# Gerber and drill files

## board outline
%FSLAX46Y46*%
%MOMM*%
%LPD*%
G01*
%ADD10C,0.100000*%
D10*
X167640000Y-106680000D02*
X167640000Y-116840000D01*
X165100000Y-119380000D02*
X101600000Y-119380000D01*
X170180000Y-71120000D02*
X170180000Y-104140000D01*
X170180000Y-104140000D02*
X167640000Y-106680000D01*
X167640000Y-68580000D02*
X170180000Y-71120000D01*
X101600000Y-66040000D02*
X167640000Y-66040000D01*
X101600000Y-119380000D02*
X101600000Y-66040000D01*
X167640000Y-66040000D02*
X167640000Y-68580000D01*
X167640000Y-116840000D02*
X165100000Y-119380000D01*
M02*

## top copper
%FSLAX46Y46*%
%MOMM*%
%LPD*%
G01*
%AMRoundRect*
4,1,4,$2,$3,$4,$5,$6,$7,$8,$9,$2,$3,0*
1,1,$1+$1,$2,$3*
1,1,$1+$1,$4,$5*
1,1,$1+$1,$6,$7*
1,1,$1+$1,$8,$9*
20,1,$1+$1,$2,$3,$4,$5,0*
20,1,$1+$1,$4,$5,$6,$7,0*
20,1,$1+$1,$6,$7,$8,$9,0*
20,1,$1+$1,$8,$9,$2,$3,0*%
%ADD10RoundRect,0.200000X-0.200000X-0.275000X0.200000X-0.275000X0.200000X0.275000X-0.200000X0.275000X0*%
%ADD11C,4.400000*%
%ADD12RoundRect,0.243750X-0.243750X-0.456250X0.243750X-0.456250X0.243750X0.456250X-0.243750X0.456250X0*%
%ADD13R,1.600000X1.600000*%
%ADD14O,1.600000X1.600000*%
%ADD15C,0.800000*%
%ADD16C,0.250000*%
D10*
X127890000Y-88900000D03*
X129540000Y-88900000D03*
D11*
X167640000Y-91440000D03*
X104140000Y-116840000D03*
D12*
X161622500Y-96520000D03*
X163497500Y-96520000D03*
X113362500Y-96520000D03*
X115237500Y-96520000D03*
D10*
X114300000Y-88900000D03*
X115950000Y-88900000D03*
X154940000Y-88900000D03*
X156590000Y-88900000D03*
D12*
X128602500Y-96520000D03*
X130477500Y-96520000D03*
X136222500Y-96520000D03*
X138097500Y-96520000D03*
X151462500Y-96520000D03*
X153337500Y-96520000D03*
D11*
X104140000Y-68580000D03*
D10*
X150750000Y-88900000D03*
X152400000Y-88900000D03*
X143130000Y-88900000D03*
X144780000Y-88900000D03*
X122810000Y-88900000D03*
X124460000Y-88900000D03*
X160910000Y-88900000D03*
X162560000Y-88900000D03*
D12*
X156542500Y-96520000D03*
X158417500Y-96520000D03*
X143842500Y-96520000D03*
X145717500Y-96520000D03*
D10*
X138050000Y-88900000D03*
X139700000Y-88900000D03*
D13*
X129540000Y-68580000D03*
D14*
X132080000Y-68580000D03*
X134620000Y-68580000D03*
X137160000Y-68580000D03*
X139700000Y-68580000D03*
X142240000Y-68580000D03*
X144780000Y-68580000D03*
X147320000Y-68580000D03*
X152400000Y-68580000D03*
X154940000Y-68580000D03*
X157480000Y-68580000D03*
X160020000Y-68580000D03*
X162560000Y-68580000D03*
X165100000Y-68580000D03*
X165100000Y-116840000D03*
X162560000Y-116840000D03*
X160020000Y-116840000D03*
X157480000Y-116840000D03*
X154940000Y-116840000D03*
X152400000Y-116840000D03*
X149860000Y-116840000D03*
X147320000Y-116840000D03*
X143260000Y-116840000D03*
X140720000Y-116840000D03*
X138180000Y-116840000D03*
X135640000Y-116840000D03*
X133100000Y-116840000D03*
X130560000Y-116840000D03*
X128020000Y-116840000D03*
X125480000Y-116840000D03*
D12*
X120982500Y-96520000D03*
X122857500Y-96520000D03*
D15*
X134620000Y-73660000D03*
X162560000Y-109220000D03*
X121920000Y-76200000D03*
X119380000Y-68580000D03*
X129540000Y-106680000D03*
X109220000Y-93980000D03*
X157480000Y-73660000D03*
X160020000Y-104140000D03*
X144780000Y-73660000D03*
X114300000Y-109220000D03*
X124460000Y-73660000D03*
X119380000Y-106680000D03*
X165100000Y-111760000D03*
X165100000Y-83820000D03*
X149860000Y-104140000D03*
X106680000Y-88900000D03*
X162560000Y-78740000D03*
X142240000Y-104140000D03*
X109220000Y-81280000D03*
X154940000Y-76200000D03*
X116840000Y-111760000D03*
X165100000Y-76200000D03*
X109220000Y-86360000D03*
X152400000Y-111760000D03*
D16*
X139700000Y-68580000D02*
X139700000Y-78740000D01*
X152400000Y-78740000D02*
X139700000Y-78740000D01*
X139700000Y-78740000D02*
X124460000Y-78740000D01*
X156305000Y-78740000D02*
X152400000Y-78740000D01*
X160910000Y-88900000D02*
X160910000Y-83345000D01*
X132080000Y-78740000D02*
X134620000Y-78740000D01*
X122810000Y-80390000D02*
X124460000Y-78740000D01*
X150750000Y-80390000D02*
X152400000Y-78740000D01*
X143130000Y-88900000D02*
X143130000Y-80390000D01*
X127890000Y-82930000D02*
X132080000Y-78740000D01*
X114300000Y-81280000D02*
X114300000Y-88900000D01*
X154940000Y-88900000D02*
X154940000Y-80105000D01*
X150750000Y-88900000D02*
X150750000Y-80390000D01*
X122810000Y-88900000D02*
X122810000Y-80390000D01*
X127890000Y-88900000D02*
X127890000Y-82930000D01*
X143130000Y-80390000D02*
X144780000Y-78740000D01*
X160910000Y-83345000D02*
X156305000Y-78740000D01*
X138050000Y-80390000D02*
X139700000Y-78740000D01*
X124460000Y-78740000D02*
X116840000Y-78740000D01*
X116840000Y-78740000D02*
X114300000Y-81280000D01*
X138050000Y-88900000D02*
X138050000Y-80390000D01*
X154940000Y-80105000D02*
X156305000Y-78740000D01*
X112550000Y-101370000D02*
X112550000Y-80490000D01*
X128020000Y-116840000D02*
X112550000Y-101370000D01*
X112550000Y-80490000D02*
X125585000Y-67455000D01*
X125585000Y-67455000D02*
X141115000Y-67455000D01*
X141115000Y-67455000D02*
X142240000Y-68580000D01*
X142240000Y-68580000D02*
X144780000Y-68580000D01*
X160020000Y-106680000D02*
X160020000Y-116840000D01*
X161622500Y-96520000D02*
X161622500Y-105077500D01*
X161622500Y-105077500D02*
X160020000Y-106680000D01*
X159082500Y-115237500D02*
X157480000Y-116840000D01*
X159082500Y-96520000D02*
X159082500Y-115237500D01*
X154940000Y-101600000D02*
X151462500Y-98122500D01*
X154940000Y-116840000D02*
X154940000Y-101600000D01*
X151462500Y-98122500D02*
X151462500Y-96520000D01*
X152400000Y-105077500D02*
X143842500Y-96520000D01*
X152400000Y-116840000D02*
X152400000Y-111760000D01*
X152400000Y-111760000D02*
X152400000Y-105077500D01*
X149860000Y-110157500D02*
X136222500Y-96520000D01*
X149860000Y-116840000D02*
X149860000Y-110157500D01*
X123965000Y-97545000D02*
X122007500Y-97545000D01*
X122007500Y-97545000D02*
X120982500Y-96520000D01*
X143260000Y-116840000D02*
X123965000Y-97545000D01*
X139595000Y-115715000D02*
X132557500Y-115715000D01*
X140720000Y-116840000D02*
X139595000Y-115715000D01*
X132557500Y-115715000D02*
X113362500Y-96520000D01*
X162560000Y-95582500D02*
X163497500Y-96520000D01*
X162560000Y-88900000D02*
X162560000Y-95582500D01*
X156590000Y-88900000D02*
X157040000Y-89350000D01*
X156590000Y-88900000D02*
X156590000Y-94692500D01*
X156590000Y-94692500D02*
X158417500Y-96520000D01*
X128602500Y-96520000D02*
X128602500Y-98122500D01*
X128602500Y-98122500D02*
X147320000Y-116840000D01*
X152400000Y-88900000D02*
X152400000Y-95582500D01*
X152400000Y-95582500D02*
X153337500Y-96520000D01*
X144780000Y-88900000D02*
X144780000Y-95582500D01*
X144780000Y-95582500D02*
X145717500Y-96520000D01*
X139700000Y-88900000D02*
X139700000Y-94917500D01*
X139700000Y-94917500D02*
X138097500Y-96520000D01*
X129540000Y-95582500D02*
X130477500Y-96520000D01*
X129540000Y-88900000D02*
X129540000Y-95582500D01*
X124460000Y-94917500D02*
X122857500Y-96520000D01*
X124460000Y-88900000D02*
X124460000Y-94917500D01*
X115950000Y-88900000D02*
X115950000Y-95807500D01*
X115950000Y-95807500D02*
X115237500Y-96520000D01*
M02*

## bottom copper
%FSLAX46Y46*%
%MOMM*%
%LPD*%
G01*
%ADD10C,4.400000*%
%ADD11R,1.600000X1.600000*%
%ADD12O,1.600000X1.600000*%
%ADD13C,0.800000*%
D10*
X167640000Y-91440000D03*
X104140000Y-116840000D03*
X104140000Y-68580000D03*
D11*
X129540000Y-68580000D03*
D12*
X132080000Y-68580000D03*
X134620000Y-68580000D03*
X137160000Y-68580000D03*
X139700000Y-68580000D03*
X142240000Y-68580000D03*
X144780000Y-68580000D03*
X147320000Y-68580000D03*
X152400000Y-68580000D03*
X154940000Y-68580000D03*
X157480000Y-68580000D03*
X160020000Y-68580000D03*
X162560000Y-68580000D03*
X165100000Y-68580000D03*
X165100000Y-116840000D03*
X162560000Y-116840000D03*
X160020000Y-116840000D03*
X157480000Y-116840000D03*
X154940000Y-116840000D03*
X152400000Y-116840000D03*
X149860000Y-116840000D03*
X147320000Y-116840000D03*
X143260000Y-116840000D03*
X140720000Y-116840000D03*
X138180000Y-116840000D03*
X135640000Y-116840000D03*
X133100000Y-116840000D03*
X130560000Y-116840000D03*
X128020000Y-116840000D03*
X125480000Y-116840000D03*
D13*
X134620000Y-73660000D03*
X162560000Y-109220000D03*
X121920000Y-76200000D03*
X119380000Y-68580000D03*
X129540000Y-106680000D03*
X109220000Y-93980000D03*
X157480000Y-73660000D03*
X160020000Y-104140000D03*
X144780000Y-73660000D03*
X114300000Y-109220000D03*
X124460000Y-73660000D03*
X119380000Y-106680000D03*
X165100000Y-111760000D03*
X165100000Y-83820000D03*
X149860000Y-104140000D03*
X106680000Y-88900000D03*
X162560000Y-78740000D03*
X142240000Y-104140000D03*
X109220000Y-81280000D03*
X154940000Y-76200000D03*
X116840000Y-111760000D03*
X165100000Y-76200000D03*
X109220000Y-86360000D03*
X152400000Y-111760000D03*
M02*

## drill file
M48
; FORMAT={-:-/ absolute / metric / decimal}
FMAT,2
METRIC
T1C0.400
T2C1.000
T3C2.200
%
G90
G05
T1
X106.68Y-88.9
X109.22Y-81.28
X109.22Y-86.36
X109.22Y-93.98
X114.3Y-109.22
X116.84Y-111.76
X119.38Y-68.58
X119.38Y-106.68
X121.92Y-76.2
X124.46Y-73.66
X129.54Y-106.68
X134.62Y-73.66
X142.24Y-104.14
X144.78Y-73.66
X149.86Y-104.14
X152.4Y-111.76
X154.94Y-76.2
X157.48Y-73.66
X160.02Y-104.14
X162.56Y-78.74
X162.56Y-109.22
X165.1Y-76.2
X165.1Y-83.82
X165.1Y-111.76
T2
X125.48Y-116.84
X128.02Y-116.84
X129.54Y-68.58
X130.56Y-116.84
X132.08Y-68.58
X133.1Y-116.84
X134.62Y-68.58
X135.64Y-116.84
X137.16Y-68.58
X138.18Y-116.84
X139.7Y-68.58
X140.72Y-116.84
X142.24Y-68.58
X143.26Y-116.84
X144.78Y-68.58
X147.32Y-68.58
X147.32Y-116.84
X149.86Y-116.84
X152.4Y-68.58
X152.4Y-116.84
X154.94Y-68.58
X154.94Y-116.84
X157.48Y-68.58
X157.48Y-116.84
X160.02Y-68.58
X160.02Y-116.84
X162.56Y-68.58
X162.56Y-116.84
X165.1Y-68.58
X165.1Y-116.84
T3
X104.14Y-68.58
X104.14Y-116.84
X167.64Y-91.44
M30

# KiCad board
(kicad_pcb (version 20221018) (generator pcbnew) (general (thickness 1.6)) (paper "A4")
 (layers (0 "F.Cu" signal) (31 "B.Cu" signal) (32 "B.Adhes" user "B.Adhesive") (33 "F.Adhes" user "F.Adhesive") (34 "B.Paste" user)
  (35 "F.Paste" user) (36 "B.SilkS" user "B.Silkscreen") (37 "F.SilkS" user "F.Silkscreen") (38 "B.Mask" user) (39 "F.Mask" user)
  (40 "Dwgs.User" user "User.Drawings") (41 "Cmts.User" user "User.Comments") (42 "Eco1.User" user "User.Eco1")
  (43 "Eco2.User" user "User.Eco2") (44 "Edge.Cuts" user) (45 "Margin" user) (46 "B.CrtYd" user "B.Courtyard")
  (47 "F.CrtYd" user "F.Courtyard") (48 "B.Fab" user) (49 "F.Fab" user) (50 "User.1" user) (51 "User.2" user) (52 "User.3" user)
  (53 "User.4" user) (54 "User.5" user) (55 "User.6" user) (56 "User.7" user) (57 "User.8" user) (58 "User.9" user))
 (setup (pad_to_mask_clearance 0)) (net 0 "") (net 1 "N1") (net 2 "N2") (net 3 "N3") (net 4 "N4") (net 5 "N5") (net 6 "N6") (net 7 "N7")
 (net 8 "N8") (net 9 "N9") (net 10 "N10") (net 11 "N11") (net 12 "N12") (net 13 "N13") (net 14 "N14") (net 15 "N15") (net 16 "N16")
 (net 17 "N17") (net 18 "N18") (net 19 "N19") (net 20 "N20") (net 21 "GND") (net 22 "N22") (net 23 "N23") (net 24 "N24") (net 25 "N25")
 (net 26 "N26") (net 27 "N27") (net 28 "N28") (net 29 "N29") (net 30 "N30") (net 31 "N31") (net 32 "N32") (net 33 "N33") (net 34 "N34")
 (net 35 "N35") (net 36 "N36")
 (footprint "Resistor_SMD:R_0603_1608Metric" (layer "F.Cu") (at 128.715 88.9)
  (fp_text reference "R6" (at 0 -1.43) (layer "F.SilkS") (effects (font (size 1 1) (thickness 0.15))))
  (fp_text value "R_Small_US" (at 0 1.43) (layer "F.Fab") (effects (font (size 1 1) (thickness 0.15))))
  (pad "1" smd roundrect (at -0.825 0) (size 0.8 0.95) (layers "F.Cu" "F.Paste" "F.Mask") (roundrect_rratio 0.25) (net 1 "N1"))
  (pad "2" smd roundrect (at 0.825 0) (size 0.8 0.95) (layers "F.Cu" "F.Paste" "F.Mask") (roundrect_rratio 0.25) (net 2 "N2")))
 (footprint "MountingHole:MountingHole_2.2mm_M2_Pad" (layer "F.Cu") (at 167.64 91.44)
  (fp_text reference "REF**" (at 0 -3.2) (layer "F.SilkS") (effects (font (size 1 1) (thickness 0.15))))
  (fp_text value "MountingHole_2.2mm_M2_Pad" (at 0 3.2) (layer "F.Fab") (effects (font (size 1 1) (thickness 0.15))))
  (pad "1" thru_hole circle (at 0 0) (size 4.4 4.4) (drill 2.2) (layers "*.Cu" "*.Mask")))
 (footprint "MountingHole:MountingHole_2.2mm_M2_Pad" (layer "F.Cu") (at 104.14 116.84)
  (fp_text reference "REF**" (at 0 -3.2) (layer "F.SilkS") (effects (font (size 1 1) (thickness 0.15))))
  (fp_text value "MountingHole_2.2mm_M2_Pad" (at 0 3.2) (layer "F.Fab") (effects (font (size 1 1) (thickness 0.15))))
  (pad "1" thru_hole circle (at 0 0) (size 4.4 4.4) (drill 2.2) (layers "*.Cu" "*.Mask")))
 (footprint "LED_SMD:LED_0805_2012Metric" (layer "F.Cu") (at 162.56 96.52)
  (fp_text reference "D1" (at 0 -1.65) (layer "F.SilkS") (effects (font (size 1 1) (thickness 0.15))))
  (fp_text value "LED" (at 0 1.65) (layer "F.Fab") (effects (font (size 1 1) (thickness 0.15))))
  (pad "1" smd roundrect (at -0.9375 0) (size 0.975 1.4) (layers "F.Cu" "F.Paste" "F.Mask") (roundrect_rratio 0.25) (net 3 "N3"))
  (pad "2" smd roundrect (at 0.9375 0) (size 0.975 1.4) (layers "F.Cu" "F.Paste" "F.Mask") (roundrect_rratio 0.25) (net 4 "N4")))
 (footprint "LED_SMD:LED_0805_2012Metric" (layer "F.Cu") (at 114.3 96.52)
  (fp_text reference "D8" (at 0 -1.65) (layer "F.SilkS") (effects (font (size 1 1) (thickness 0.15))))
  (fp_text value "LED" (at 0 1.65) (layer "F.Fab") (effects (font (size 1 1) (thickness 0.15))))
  (pad "1" smd roundrect (at -0.9375 0) (size 0.975 1.4) (layers "F.Cu" "F.Paste" "F.Mask") (roundrect_rratio 0.25) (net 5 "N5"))
  (pad "2" smd roundrect (at 0.9375 0) (size 0.975 1.4) (layers "F.Cu" "F.Paste" "F.Mask") (roundrect_rratio 0.25) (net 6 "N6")))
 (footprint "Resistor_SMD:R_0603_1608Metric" (layer "F.Cu") (at 115.125 88.9)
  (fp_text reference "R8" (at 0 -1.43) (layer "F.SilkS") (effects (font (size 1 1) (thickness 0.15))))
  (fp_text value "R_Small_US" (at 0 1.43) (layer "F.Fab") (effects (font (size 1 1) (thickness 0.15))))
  (pad "1" smd roundrect (at -0.825 0) (size 0.8 0.95) (layers "F.Cu" "F.Paste" "F.Mask") (roundrect_rratio 0.25) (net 1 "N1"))
  (pad "2" smd roundrect (at 0.825 0) (size 0.8 0.95) (layers "F.Cu" "F.Paste" "F.Mask") (roundrect_rratio 0.25) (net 6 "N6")))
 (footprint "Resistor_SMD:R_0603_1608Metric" (layer "F.Cu") (at 155.765 88.9)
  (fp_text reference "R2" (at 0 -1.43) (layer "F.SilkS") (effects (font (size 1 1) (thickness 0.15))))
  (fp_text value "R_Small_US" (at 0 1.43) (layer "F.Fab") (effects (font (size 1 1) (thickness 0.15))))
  (pad "1" smd roundrect (at -0.825 0) (size 0.8 0.95) (layers "F.Cu" "F.Paste" "F.Mask") (roundrect_rratio 0.25) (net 1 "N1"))
  (pad "2" smd roundrect (at 0.825 0) (size 0.8 0.95) (layers "F.Cu" "F.Paste" "F.Mask") (roundrect_rratio 0.25) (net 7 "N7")))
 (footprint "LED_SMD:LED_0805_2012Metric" (layer "F.Cu") (at 129.54 96.52)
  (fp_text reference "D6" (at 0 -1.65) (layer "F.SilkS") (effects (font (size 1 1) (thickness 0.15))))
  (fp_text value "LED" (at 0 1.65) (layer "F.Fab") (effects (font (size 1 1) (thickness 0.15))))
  (pad "1" smd roundrect (at -0.9375 0) (size 0.975 1.4) (layers "F.Cu" "F.Paste" "F.Mask") (roundrect_rratio 0.25) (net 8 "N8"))
  (pad "2" smd roundrect (at 0.9375 0) (size 0.975 1.4) (layers "F.Cu" "F.Paste" "F.Mask") (roundrect_rratio 0.25) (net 2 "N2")))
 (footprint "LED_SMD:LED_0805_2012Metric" (layer "F.Cu") (at 137.16 96.52)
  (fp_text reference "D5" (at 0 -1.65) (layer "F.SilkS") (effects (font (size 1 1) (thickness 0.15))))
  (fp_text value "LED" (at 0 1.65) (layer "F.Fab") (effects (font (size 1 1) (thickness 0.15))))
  (pad "1" smd roundrect (at -0.9375 0) (size 0.975 1.4) (layers "F.Cu" "F.Paste" "F.Mask") (roundrect_rratio 0.25) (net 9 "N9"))
  (pad "2" smd roundrect (at 0.9375 0) (size 0.975 1.4) (layers "F.Cu" "F.Paste" "F.Mask") (roundrect_rratio 0.25) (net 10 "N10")))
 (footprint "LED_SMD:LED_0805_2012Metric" (layer "F.Cu") (at 152.4 96.52)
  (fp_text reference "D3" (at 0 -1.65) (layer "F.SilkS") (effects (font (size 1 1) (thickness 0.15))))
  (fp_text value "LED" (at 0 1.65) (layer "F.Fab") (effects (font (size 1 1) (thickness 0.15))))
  (pad "1" smd roundrect (at -0.9375 0) (size 0.975 1.4) (layers "F.Cu" "F.Paste" "F.Mask") (roundrect_rratio 0.25) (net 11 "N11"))
  (pad "2" smd roundrect (at 0.9375 0) (size 0.975 1.4) (layers "F.Cu" "F.Paste" "F.Mask") (roundrect_rratio 0.25) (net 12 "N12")))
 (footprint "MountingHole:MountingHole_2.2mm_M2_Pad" (layer "F.Cu") (at 104.14 68.58)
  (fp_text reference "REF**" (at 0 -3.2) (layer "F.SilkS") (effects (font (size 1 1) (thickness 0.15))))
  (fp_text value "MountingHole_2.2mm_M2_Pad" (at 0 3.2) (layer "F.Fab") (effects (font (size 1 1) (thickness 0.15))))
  (pad "1" thru_hole circle (at 0 0) (size 4.4 4.4) (drill 2.2) (layers "*.Cu" "*.Mask")))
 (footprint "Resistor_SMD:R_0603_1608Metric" (layer "F.Cu") (at 151.575 88.9)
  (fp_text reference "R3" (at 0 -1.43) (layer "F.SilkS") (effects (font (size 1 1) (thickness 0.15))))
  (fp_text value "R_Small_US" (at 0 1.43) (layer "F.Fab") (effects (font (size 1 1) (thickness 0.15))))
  (pad "1" smd roundrect (at -0.825 0) (size 0.8 0.95) (layers "F.Cu" "F.Paste" "F.Mask") (roundrect_rratio 0.25) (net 1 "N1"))
  (pad "2" smd roundrect (at 0.825 0) (size 0.8 0.95) (layers "F.Cu" "F.Paste" "F.Mask") (roundrect_rratio 0.25) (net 12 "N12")))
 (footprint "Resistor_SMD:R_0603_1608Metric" (layer "F.Cu") (at 143.955 88.9)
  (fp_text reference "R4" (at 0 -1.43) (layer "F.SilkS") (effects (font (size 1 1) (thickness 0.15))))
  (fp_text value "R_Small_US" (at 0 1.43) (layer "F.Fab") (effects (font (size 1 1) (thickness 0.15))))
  (pad "1" smd roundrect (at -0.825 0) (size 0.8 0.95) (layers "F.Cu" "F.Paste" "F.Mask") (roundrect_rratio 0.25) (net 1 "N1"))
  (pad "2" smd roundrect (at 0.825 0) (size 0.8 0.95) (layers "F.Cu" "F.Paste" "F.Mask") (roundrect_rratio 0.25) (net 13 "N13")))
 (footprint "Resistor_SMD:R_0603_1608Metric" (layer "F.Cu") (at 123.635 88.9)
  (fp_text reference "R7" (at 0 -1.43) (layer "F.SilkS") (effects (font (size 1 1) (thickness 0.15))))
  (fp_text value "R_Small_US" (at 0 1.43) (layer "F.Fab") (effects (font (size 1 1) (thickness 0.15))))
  (pad "1" smd roundrect (at -0.825 0) (size 0.8 0.95) (layers "F.Cu" "F.Paste" "F.Mask") (roundrect_rratio 0.25) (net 1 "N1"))
  (pad "2" smd roundrect (at 0.825 0) (size 0.8 0.95) (layers "F.Cu" "F.Paste" "F.Mask") (roundrect_rratio 0.25) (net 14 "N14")))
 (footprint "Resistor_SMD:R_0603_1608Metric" (layer "F.Cu") (at 161.735 88.9)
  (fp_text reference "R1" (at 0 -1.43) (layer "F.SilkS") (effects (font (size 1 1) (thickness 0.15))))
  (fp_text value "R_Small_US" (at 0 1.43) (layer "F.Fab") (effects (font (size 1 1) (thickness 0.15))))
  (pad "1" smd roundrect (at -0.825 0) (size 0.8 0.95) (layers "F.Cu" "F.Paste" "F.Mask") (roundrect_rratio 0.25) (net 1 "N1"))
  (pad "2" smd roundrect (at 0.825 0) (size 0.8 0.95) (layers "F.Cu" "F.Paste" "F.Mask") (roundrect_rratio 0.25) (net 4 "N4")))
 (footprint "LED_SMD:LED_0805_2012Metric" (layer "F.Cu") (at 157.48 96.52)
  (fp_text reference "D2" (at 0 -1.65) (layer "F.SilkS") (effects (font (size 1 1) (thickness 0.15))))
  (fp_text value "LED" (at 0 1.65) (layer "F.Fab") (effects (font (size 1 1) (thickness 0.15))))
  (pad "1" smd roundrect (at -0.9375 0) (size 0.975 1.4) (layers "F.Cu" "F.Paste" "F.Mask") (roundrect_rratio 0.25) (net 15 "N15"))
  (pad "2" smd roundrect (at 0.9375 0) (size 0.975 1.4) (layers "F.Cu" "F.Paste" "F.Mask") (roundrect_rratio 0.25) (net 7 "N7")))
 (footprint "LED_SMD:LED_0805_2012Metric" (layer "F.Cu") (at 144.78 96.52)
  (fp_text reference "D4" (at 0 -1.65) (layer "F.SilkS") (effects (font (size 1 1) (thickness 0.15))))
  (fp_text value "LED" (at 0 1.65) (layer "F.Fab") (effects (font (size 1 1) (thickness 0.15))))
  (pad "1" smd roundrect (at -0.9375 0) (size 0.975 1.4) (layers "F.Cu" "F.Paste" "F.Mask") (roundrect_rratio 0.25) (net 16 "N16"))
  (pad "2" smd roundrect (at 0.9375 0) (size 0.975 1.4) (layers "F.Cu" "F.Paste" "F.Mask") (roundrect_rratio 0.25) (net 13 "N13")))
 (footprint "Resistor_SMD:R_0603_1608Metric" (layer "F.Cu") (at 138.875 88.9)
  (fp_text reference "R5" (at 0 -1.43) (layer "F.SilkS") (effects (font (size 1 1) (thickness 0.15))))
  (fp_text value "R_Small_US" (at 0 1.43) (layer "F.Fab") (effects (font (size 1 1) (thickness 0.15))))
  (pad "1" smd roundrect (at -0.825 0) (size 0.8 0.95) (layers "F.Cu" "F.Paste" "F.Mask") (roundrect_rratio 0.25) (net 1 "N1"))
  (pad "2" smd roundrect (at 0.825 0) (size 0.8 0.95) (layers "F.Cu" "F.Paste" "F.Mask") (roundrect_rratio 0.25) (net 10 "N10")))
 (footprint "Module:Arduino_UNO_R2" (layer "F.Cu") (at 129.54 68.58)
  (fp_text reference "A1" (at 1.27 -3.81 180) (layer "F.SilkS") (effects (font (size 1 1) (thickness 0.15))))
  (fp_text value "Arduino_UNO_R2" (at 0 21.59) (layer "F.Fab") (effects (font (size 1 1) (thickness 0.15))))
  (pad "1" thru_hole rect (at 0 0 90) (size 1.6 1.6) (drill 1) (layers "*.Cu" "*.Mask") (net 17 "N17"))
  (pad "2" thru_hole oval (at 2.54 0 90) (size 1.6 1.6) (drill 1) (layers "*.Cu" "*.Mask") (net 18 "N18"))
  (pad "3" thru_hole oval (at 5.08 0 90) (size 1.6 1.6) (drill 1) (layers "*.Cu" "*.Mask") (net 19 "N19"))
  (pad "4" thru_hole oval (at 7.62 0 90) (size 1.6 1.6) (drill 1) (layers "*.Cu" "*.Mask") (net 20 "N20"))
  (pad "5" thru_hole oval (at 10.16 0 90) (size 1.6 1.6) (drill 1) (layers "*.Cu" "*.Mask") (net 1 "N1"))
  (pad "6" thru_hole oval (at 12.7 0 90) (size 1.6 1.6) (drill 1) (layers "*.Cu" "*.Mask") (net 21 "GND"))
  (pad "7" thru_hole oval (at 15.24 0 90) (size 1.6 1.6) (drill 1) (layers "*.Cu" "*.Mask") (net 21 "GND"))
  (pad "8" thru_hole oval (at 17.78 0 90) (size 1.6 1.6) (drill 1) (layers "*.Cu" "*.Mask") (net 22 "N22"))
  (pad "9" thru_hole oval (at 22.86 0 90) (size 1.6 1.6) (drill 1) (layers "*.Cu" "*.Mask") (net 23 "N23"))
  (pad "10" thru_hole oval (at 25.4 0 90) (size 1.6 1.6) (drill 1) (layers "*.Cu" "*.Mask") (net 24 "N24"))
  (pad "11" thru_hole oval (at 27.94 0 90) (size 1.6 1.6) (drill 1) (layers "*.Cu" "*.Mask") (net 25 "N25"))
  (pad "12" thru_hole oval (at 30.48 0 90) (size 1.6 1.6) (drill 1) (layers "*.Cu" "*.Mask") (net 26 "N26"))
  (pad "13" thru_hole oval (at 33.02 0 90) (size 1.6 1.6) (drill 1) (layers "*.Cu" "*.Mask") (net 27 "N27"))
  (pad "14" thru_hole oval (at 35.56 0 90) (size 1.6 1.6) (drill 1) (layers "*.Cu" "*.Mask") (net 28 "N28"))
  (pad "15" thru_hole oval (at 35.56 48.26 90) (size 1.6 1.6) (drill 1) (layers "*.Cu" "*.Mask") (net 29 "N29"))
  (pad "16" thru_hole oval (at 33.02 48.26 90) (size 1.6 1.6) (drill 1) (layers "*.Cu" "*.Mask") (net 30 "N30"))
  (pad "17" thru_hole oval (at 30.48 48.26 90) (size 1.6 1.6) (drill 1) (layers "*.Cu" "*.Mask") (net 3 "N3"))
  (pad "18" thru_hole oval (at 27.94 48.26 90) (size 1.6 1.6) (drill 1) (layers "*.Cu" "*.Mask") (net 15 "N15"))
  (pad "19" thru_hole oval (at 25.4 48.26 90) (size 1.6 1.6) (drill 1) (layers "*.Cu" "*.Mask") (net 11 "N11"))
  (pad "20" thru_hole oval (at 22.86 48.26 90) (size 1.6 1.6) (drill 1) (layers "*.Cu" "*.Mask") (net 16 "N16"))
  (pad "21" thru_hole oval (at 20.32 48.26 90) (size 1.6 1.6) (drill 1) (layers "*.Cu" "*.Mask") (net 9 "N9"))
  (pad "22" thru_hole oval (at 17.78 48.26 90) (size 1.6 1.6) (drill 1) (layers "*.Cu" "*.Mask") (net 8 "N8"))
  (pad "23" thru_hole oval (at 13.72 48.26 90) (size 1.6 1.6) (drill 1) (layers "*.Cu" "*.Mask") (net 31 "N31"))
  (pad "24" thru_hole oval (at 11.18 48.26 90) (size 1.6 1.6) (drill 1) (layers "*.Cu" "*.Mask") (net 5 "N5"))
  (pad "25" thru_hole oval (at 8.64 48.26 90) (size 1.6 1.6) (drill 1) (layers "*.Cu" "*.Mask") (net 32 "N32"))
  (pad "26" thru_hole oval (at 6.1 48.26 90) (size 1.6 1.6) (drill 1) (layers "*.Cu" "*.Mask") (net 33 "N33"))
  (pad "27" thru_hole oval (at 3.56 48.26 90) (size 1.6 1.6) (drill 1) (layers "*.Cu" "*.Mask") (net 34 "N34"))
  (pad "28" thru_hole oval (at 1.02 48.26 90) (size 1.6 1.6) (drill 1) (layers "*.Cu" "*.Mask") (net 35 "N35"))
  (pad "29" thru_hole oval (at -1.52 48.26 90) (size 1.6 1.6) (drill 1) (layers "*.Cu" "*.Mask") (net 21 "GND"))
  (pad "30" thru_hole oval (at -4.06 48.26 90) (size 1.6 1.6) (drill 1) (layers "*.Cu" "*.Mask") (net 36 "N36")))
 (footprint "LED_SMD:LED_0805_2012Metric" (layer "F.Cu") (at 121.92 96.52)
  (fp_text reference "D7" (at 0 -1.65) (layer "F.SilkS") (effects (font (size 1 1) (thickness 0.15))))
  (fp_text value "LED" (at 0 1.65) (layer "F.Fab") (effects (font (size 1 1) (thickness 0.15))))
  (pad "1" smd roundrect (at -0.9375 0) (size 0.975 1.4) (layers "F.Cu" "F.Paste" "F.Mask") (roundrect_rratio 0.25) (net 31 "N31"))
  (pad "2" smd roundrect (at 0.9375 0) (size 0.975 1.4) (layers "F.Cu" "F.Paste" "F.Mask") (roundrect_rratio 0.25) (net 14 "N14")))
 (gr_line (start 167.64 106.68) (end 167.64 116.84) (stroke (width 0.1) (type default)) (layer "Edge.Cuts"))
 (gr_line (start 165.1 119.38) (end 101.6 119.38) (stroke (width 0.1) (type default)) (layer "Edge.Cuts"))
 (gr_line (start 170.18 71.12) (end 170.18 104.14) (stroke (width 0.1) (type default)) (layer "Edge.Cuts"))
 (gr_line (start 170.18 104.14) (end 167.64 106.68) (stroke (width 0.1) (type default)) (layer "Edge.Cuts"))
 (gr_line (start 167.64 68.58) (end 170.18 71.12) (stroke (width 0.1) (type default)) (layer "Edge.Cuts"))
 (gr_line (start 101.6 66.04) (end 167.64 66.04) (stroke (width 0.1) (type default)) (layer "Edge.Cuts"))
 (gr_line (start 101.6 119.38) (end 101.6 66.04) (stroke (width 0.1) (type default)) (layer "Edge.Cuts"))
 (gr_line (start 167.64 66.04) (end 167.64 68.58) (stroke (width 0.1) (type default)) (layer "Edge.Cuts"))
 (gr_line (start 167.64 116.84) (end 165.1 119.38) (stroke (width 0.1) (type default)) (layer "Edge.Cuts"))
 (via (at 134.62 73.66) (size 0.8) (drill 0.4) (layers "F.Cu" "B.Cu") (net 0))
 (via (at 162.56 109.22) (size 0.8) (drill 0.4) (layers "F.Cu" "B.Cu") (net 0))
 (via (at 121.92 76.2) (size 0.8) (drill 0.4) (layers "F.Cu" "B.Cu") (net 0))
 (via (at 119.38 68.58) (size 0.8) (drill 0.4) (layers "F.Cu" "B.Cu") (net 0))
 (via (at 129.54 106.68) (size 0.8) (drill 0.4) (layers "F.Cu" "B.Cu") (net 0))
 (via (at 109.22 93.98) (size 0.8) (drill 0.4) (layers "F.Cu" "B.Cu") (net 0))
 (via (at 157.48 73.66) (size 0.8) (drill 0.4) (layers "F.Cu" "B.Cu") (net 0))
 (via (at 160.02 104.14) (size 0.8) (drill 0.4) (layers "F.Cu" "B.Cu") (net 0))
 (via (at 144.78 73.66) (size 0.8) (drill 0.4) (layers "F.Cu" "B.Cu") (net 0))
 (via (at 114.3 109.22) (size 0.8) (drill 0.4) (layers "F.Cu" "B.Cu") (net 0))
 (via (at 124.46 73.66) (size 0.8) (drill 0.4) (layers "F.Cu" "B.Cu") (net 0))
 (via (at 119.38 106.68) (size 0.8) (drill 0.4) (layers "F.Cu" "B.Cu") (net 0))
 (via (at 165.1 111.76) (size 0.8) (drill 0.4) (layers "F.Cu" "B.Cu") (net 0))
 (via (at 165.1 83.82) (size 0.8) (drill 0.4) (layers "F.Cu" "B.Cu") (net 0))
 (via (at 149.86 104.14) (size 0.8) (drill 0.4) (layers "F.Cu" "B.Cu") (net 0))
 (via (at 106.68 88.9) (size 0.8) (drill 0.4) (layers "F.Cu" "B.Cu") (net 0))
 (via (at 162.56 78.74) (size 0.8) (drill 0.4) (layers "F.Cu" "B.Cu") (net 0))
 (via (at 142.24 104.14) (size 0.8) (drill 0.4) (layers "F.Cu" "B.Cu") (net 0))
 (via (at 109.22 81.28) (size 0.8) (drill 0.4) (layers "F.Cu" "B.Cu") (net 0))
 (via (at 154.94 76.2) (size 0.8) (drill 0.4) (layers "F.Cu" "B.Cu") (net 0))
 (via (at 116.84 111.76) (size 0.8) (drill 0.4) (layers "F.Cu" "B.Cu") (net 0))
 (via (at 165.1 76.2) (size 0.8) (drill 0.4) (layers "F.Cu" "B.Cu") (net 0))
 (via (at 109.22 86.36) (size 0.8) (drill 0.4) (layers "F.Cu" "B.Cu") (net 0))
 (segment (start 139.7 68.58) (end 139.7 78.74) (width 0.25) (layer "F.Cu") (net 1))
 (segment (start 152.4 78.74) (end 139.7 78.74) (width 0.25) (layer "F.Cu") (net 1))
 (segment (start 139.7 78.74) (end 124.46 78.74) (width 0.25) (layer "F.Cu") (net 1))
 (segment (start 156.305 78.74) (end 152.4 78.74) (width 0.25) (layer "F.Cu") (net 1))
 (segment (start 160.91 88.9) (end 160.91 83.345) (width 0.25) (layer "F.Cu") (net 1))
 (segment (start 132.08 78.74) (end 134.62 78.74) (width 0.25) (layer "F.Cu") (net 1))
 (segment (start 122.81 80.39) (end 124.46 78.74) (width 0.25) (layer "F.Cu") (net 1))
 (segment (start 150.75 80.39) (end 152.4 78.74) (width 0.25) (layer "F.Cu") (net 1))
 (segment (start 143.13 88.9) (end 143.13 80.39) (width 0.25) (layer "F.Cu") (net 1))
 (segment (start 127.89 82.93) (end 132.08 78.74) (width 0.25) (layer "F.Cu") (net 1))
 (segment (start 114.3 81.28) (end 114.3 88.9) (width 0.25) (layer "F.Cu") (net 1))
 (segment (start 154.94 88.9) (end 154.94 80.105) (width 0.25) (layer "F.Cu") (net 1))
 (segment (start 150.75 88.9) (end 150.75 80.39) (width 0.25) (layer "F.Cu") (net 1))
 (segment (start 122.81 88.9) (end 122.81 80.39) (width 0.25) (layer "F.Cu") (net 1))
 (segment (start 127.89 88.9) (end 127.89 82.93) (width 0.25) (layer "F.Cu") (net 1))
 (segment (start 143.13 80.39) (end 144.78 78.74) (width 0.25) (layer "F.Cu") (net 1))
 (segment (start 160.91 83.345) (end 156.305 78.74) (width 0.25) (layer "F.Cu") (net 1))
 (segment (start 138.05 80.39) (end 139.7 78.74) (width 0.25) (layer "F.Cu") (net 1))
 (segment (start 124.46 78.74) (end 116.84 78.74) (width 0.25) (layer "F.Cu") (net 1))
 (segment (start 116.84 78.74) (end 114.3 81.28) (width 0.25) (layer "F.Cu") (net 1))
 (segment (start 138.05 88.9) (end 138.05 80.39) (width 0.25) (layer "F.Cu") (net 1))
 (segment (start 154.94 80.105) (end 156.305 78.74) (width 0.25) (layer "F.Cu") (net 1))
 (segment (start 112.55 101.37) (end 112.55 80.49) (width 0.25) (layer "F.Cu") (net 21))
 (segment (start 128.02 116.84) (end 112.55 101.37) (width 0.25) (layer "F.Cu") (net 21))
 (segment (start 112.55 80.49) (end 125.585 67.455) (width 0.25) (layer "F.Cu") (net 21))
 (segment (start 125.585 67.455) (end 141.115 67.455) (width 0.25) (layer "F.Cu") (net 21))
 (segment (start 141.115 67.455) (end 142.24 68.58) (width 0.25) (layer "F.Cu") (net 21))
 (segment (start 142.24 68.58) (end 144.78 68.58) (width 0.25) (layer "F.Cu") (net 21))
 (segment (start 160.02 106.68) (end 160.02 116.84) (width 0.25) (layer "F.Cu") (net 3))
 (segment (start 161.6225 96.52) (end 161.6225 105.0775) (width 0.25) (layer "F.Cu") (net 3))
 (segment (start 161.6225 105.0775) (end 160.02 106.68) (width 0.25) (layer "F.Cu") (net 3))
 (segment (start 159.0825 115.2375) (end 157.48 116.84) (width 0.25) (layer "F.Cu") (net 15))
 (segment (start 159.0825 96.52) (end 159.0825 115.2375) (width 0.25) (layer "F.Cu") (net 15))
 (segment (start 154.94 101.6) (end 151.4625 98.1225) (width 0.25) (layer "F.Cu") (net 11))
 (segment (start 154.94 116.84) (end 154.94 101.6) (width 0.25) (layer "F.Cu") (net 11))
 (segment (start 151.4625 98.1225) (end 151.4625 96.52) (width 0.25) (layer "F.Cu") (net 11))
 (segment (start 152.4 105.0775) (end 143.8425 96.52) (width 0.25) (layer "F.Cu") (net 16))
 (segment (start 152.4 116.84) (end 152.4 111.76) (width 0.25) (layer "F.Cu") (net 16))
 (segment (start 152.4 111.76) (end 152.4 105.0775) (width 0.25) (layer "F.Cu") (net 16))
 (via (at 152.4 111.76) (size 0.8) (drill 0.4) (layers "F.Cu" "B.Cu") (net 16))
 (segment (start 149.86 110.1575) (end 136.2225 96.52) (width 0.25) (layer "F.Cu") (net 9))
 (segment (start 149.86 116.84) (end 149.86 110.1575) (width 0.25) (layer "F.Cu") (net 9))
 (segment (start 123.965 97.545) (end 122.0075 97.545) (width 0.25) (layer "F.Cu") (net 31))
 (segment (start 122.0075 97.545) (end 120.9825 96.52) (width 0.25) (layer "F.Cu") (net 31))
 (segment (start 143.26 116.84) (end 123.965 97.545) (width 0.25) (layer "F.Cu") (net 31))
 (segment (start 139.595 115.715) (end 132.5575 115.715) (width 0.25) (layer "F.Cu") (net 5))
 (segment (start 140.72 116.84) (end 139.595 115.715) (width 0.25) (layer "F.Cu") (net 5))
 (segment (start 132.5575 115.715) (end 113.3625 96.52) (width 0.25) (layer "F.Cu") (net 5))
 (segment (start 162.56 95.5825) (end 163.4975 96.52) (width 0.25) (layer "F.Cu") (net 4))
 (segment (start 162.56 88.9) (end 162.56 95.5825) (width 0.25) (layer "F.Cu") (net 4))
 (segment (start 156.59 88.9) (end 157.04 89.35) (width 0.25) (layer "F.Cu") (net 7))
 (segment (start 156.59 88.9) (end 156.59 94.6925) (width 0.25) (layer "F.Cu") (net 7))
 (segment (start 156.59 94.6925) (end 158.4175 96.52) (width 0.25) (layer "F.Cu") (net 7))
 (segment (start 128.6025 96.52) (end 128.6025 98.1225) (width 0.25) (layer "F.Cu") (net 8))
 (segment (start 128.6025 98.1225) (end 147.32 116.84) (width 0.25) (layer "F.Cu") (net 8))
 (segment (start 152.4 88.9) (end 152.4 95.5825) (width 0.25) (layer "F.Cu") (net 12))
 (segment (start 152.4 95.5825) (end 153.3375 96.52) (width 0.25) (layer "F.Cu") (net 12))
 (segment (start 144.78 88.9) (end 144.78 95.5825) (width 0.25) (layer "F.Cu") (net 13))
 (segment (start 144.78 95.5825) (end 145.7175 96.52) (width 0.25) (layer "F.Cu") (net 13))
 (segment (start 139.7 88.9) (end 139.7 94.9175) (width 0.25) (layer "F.Cu") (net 10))
 (segment (start 139.7 94.9175) (end 138.0975 96.52) (width 0.25) (layer "F.Cu") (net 10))
 (segment (start 129.54 95.5825) (end 130.4775 96.52) (width 0.25) (layer "F.Cu") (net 2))
 (segment (start 129.54 88.9) (end 129.54 95.5825) (width 0.25) (layer "F.Cu") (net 2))
 (segment (start 124.46 94.9175) (end 122.8575 96.52) (width 0.25) (layer "F.Cu") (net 14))
 (segment (start 124.46 88.9) (end 124.46 94.9175) (width 0.25) (layer "F.Cu") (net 14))
 (segment (start 115.95 88.9) (end 115.95 95.8075) (width 0.25) (layer "F.Cu") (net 6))
 (segment (start 115.95 95.8075) (end 115.2375 96.52) (width 0.25) (layer "F.Cu") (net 6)))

